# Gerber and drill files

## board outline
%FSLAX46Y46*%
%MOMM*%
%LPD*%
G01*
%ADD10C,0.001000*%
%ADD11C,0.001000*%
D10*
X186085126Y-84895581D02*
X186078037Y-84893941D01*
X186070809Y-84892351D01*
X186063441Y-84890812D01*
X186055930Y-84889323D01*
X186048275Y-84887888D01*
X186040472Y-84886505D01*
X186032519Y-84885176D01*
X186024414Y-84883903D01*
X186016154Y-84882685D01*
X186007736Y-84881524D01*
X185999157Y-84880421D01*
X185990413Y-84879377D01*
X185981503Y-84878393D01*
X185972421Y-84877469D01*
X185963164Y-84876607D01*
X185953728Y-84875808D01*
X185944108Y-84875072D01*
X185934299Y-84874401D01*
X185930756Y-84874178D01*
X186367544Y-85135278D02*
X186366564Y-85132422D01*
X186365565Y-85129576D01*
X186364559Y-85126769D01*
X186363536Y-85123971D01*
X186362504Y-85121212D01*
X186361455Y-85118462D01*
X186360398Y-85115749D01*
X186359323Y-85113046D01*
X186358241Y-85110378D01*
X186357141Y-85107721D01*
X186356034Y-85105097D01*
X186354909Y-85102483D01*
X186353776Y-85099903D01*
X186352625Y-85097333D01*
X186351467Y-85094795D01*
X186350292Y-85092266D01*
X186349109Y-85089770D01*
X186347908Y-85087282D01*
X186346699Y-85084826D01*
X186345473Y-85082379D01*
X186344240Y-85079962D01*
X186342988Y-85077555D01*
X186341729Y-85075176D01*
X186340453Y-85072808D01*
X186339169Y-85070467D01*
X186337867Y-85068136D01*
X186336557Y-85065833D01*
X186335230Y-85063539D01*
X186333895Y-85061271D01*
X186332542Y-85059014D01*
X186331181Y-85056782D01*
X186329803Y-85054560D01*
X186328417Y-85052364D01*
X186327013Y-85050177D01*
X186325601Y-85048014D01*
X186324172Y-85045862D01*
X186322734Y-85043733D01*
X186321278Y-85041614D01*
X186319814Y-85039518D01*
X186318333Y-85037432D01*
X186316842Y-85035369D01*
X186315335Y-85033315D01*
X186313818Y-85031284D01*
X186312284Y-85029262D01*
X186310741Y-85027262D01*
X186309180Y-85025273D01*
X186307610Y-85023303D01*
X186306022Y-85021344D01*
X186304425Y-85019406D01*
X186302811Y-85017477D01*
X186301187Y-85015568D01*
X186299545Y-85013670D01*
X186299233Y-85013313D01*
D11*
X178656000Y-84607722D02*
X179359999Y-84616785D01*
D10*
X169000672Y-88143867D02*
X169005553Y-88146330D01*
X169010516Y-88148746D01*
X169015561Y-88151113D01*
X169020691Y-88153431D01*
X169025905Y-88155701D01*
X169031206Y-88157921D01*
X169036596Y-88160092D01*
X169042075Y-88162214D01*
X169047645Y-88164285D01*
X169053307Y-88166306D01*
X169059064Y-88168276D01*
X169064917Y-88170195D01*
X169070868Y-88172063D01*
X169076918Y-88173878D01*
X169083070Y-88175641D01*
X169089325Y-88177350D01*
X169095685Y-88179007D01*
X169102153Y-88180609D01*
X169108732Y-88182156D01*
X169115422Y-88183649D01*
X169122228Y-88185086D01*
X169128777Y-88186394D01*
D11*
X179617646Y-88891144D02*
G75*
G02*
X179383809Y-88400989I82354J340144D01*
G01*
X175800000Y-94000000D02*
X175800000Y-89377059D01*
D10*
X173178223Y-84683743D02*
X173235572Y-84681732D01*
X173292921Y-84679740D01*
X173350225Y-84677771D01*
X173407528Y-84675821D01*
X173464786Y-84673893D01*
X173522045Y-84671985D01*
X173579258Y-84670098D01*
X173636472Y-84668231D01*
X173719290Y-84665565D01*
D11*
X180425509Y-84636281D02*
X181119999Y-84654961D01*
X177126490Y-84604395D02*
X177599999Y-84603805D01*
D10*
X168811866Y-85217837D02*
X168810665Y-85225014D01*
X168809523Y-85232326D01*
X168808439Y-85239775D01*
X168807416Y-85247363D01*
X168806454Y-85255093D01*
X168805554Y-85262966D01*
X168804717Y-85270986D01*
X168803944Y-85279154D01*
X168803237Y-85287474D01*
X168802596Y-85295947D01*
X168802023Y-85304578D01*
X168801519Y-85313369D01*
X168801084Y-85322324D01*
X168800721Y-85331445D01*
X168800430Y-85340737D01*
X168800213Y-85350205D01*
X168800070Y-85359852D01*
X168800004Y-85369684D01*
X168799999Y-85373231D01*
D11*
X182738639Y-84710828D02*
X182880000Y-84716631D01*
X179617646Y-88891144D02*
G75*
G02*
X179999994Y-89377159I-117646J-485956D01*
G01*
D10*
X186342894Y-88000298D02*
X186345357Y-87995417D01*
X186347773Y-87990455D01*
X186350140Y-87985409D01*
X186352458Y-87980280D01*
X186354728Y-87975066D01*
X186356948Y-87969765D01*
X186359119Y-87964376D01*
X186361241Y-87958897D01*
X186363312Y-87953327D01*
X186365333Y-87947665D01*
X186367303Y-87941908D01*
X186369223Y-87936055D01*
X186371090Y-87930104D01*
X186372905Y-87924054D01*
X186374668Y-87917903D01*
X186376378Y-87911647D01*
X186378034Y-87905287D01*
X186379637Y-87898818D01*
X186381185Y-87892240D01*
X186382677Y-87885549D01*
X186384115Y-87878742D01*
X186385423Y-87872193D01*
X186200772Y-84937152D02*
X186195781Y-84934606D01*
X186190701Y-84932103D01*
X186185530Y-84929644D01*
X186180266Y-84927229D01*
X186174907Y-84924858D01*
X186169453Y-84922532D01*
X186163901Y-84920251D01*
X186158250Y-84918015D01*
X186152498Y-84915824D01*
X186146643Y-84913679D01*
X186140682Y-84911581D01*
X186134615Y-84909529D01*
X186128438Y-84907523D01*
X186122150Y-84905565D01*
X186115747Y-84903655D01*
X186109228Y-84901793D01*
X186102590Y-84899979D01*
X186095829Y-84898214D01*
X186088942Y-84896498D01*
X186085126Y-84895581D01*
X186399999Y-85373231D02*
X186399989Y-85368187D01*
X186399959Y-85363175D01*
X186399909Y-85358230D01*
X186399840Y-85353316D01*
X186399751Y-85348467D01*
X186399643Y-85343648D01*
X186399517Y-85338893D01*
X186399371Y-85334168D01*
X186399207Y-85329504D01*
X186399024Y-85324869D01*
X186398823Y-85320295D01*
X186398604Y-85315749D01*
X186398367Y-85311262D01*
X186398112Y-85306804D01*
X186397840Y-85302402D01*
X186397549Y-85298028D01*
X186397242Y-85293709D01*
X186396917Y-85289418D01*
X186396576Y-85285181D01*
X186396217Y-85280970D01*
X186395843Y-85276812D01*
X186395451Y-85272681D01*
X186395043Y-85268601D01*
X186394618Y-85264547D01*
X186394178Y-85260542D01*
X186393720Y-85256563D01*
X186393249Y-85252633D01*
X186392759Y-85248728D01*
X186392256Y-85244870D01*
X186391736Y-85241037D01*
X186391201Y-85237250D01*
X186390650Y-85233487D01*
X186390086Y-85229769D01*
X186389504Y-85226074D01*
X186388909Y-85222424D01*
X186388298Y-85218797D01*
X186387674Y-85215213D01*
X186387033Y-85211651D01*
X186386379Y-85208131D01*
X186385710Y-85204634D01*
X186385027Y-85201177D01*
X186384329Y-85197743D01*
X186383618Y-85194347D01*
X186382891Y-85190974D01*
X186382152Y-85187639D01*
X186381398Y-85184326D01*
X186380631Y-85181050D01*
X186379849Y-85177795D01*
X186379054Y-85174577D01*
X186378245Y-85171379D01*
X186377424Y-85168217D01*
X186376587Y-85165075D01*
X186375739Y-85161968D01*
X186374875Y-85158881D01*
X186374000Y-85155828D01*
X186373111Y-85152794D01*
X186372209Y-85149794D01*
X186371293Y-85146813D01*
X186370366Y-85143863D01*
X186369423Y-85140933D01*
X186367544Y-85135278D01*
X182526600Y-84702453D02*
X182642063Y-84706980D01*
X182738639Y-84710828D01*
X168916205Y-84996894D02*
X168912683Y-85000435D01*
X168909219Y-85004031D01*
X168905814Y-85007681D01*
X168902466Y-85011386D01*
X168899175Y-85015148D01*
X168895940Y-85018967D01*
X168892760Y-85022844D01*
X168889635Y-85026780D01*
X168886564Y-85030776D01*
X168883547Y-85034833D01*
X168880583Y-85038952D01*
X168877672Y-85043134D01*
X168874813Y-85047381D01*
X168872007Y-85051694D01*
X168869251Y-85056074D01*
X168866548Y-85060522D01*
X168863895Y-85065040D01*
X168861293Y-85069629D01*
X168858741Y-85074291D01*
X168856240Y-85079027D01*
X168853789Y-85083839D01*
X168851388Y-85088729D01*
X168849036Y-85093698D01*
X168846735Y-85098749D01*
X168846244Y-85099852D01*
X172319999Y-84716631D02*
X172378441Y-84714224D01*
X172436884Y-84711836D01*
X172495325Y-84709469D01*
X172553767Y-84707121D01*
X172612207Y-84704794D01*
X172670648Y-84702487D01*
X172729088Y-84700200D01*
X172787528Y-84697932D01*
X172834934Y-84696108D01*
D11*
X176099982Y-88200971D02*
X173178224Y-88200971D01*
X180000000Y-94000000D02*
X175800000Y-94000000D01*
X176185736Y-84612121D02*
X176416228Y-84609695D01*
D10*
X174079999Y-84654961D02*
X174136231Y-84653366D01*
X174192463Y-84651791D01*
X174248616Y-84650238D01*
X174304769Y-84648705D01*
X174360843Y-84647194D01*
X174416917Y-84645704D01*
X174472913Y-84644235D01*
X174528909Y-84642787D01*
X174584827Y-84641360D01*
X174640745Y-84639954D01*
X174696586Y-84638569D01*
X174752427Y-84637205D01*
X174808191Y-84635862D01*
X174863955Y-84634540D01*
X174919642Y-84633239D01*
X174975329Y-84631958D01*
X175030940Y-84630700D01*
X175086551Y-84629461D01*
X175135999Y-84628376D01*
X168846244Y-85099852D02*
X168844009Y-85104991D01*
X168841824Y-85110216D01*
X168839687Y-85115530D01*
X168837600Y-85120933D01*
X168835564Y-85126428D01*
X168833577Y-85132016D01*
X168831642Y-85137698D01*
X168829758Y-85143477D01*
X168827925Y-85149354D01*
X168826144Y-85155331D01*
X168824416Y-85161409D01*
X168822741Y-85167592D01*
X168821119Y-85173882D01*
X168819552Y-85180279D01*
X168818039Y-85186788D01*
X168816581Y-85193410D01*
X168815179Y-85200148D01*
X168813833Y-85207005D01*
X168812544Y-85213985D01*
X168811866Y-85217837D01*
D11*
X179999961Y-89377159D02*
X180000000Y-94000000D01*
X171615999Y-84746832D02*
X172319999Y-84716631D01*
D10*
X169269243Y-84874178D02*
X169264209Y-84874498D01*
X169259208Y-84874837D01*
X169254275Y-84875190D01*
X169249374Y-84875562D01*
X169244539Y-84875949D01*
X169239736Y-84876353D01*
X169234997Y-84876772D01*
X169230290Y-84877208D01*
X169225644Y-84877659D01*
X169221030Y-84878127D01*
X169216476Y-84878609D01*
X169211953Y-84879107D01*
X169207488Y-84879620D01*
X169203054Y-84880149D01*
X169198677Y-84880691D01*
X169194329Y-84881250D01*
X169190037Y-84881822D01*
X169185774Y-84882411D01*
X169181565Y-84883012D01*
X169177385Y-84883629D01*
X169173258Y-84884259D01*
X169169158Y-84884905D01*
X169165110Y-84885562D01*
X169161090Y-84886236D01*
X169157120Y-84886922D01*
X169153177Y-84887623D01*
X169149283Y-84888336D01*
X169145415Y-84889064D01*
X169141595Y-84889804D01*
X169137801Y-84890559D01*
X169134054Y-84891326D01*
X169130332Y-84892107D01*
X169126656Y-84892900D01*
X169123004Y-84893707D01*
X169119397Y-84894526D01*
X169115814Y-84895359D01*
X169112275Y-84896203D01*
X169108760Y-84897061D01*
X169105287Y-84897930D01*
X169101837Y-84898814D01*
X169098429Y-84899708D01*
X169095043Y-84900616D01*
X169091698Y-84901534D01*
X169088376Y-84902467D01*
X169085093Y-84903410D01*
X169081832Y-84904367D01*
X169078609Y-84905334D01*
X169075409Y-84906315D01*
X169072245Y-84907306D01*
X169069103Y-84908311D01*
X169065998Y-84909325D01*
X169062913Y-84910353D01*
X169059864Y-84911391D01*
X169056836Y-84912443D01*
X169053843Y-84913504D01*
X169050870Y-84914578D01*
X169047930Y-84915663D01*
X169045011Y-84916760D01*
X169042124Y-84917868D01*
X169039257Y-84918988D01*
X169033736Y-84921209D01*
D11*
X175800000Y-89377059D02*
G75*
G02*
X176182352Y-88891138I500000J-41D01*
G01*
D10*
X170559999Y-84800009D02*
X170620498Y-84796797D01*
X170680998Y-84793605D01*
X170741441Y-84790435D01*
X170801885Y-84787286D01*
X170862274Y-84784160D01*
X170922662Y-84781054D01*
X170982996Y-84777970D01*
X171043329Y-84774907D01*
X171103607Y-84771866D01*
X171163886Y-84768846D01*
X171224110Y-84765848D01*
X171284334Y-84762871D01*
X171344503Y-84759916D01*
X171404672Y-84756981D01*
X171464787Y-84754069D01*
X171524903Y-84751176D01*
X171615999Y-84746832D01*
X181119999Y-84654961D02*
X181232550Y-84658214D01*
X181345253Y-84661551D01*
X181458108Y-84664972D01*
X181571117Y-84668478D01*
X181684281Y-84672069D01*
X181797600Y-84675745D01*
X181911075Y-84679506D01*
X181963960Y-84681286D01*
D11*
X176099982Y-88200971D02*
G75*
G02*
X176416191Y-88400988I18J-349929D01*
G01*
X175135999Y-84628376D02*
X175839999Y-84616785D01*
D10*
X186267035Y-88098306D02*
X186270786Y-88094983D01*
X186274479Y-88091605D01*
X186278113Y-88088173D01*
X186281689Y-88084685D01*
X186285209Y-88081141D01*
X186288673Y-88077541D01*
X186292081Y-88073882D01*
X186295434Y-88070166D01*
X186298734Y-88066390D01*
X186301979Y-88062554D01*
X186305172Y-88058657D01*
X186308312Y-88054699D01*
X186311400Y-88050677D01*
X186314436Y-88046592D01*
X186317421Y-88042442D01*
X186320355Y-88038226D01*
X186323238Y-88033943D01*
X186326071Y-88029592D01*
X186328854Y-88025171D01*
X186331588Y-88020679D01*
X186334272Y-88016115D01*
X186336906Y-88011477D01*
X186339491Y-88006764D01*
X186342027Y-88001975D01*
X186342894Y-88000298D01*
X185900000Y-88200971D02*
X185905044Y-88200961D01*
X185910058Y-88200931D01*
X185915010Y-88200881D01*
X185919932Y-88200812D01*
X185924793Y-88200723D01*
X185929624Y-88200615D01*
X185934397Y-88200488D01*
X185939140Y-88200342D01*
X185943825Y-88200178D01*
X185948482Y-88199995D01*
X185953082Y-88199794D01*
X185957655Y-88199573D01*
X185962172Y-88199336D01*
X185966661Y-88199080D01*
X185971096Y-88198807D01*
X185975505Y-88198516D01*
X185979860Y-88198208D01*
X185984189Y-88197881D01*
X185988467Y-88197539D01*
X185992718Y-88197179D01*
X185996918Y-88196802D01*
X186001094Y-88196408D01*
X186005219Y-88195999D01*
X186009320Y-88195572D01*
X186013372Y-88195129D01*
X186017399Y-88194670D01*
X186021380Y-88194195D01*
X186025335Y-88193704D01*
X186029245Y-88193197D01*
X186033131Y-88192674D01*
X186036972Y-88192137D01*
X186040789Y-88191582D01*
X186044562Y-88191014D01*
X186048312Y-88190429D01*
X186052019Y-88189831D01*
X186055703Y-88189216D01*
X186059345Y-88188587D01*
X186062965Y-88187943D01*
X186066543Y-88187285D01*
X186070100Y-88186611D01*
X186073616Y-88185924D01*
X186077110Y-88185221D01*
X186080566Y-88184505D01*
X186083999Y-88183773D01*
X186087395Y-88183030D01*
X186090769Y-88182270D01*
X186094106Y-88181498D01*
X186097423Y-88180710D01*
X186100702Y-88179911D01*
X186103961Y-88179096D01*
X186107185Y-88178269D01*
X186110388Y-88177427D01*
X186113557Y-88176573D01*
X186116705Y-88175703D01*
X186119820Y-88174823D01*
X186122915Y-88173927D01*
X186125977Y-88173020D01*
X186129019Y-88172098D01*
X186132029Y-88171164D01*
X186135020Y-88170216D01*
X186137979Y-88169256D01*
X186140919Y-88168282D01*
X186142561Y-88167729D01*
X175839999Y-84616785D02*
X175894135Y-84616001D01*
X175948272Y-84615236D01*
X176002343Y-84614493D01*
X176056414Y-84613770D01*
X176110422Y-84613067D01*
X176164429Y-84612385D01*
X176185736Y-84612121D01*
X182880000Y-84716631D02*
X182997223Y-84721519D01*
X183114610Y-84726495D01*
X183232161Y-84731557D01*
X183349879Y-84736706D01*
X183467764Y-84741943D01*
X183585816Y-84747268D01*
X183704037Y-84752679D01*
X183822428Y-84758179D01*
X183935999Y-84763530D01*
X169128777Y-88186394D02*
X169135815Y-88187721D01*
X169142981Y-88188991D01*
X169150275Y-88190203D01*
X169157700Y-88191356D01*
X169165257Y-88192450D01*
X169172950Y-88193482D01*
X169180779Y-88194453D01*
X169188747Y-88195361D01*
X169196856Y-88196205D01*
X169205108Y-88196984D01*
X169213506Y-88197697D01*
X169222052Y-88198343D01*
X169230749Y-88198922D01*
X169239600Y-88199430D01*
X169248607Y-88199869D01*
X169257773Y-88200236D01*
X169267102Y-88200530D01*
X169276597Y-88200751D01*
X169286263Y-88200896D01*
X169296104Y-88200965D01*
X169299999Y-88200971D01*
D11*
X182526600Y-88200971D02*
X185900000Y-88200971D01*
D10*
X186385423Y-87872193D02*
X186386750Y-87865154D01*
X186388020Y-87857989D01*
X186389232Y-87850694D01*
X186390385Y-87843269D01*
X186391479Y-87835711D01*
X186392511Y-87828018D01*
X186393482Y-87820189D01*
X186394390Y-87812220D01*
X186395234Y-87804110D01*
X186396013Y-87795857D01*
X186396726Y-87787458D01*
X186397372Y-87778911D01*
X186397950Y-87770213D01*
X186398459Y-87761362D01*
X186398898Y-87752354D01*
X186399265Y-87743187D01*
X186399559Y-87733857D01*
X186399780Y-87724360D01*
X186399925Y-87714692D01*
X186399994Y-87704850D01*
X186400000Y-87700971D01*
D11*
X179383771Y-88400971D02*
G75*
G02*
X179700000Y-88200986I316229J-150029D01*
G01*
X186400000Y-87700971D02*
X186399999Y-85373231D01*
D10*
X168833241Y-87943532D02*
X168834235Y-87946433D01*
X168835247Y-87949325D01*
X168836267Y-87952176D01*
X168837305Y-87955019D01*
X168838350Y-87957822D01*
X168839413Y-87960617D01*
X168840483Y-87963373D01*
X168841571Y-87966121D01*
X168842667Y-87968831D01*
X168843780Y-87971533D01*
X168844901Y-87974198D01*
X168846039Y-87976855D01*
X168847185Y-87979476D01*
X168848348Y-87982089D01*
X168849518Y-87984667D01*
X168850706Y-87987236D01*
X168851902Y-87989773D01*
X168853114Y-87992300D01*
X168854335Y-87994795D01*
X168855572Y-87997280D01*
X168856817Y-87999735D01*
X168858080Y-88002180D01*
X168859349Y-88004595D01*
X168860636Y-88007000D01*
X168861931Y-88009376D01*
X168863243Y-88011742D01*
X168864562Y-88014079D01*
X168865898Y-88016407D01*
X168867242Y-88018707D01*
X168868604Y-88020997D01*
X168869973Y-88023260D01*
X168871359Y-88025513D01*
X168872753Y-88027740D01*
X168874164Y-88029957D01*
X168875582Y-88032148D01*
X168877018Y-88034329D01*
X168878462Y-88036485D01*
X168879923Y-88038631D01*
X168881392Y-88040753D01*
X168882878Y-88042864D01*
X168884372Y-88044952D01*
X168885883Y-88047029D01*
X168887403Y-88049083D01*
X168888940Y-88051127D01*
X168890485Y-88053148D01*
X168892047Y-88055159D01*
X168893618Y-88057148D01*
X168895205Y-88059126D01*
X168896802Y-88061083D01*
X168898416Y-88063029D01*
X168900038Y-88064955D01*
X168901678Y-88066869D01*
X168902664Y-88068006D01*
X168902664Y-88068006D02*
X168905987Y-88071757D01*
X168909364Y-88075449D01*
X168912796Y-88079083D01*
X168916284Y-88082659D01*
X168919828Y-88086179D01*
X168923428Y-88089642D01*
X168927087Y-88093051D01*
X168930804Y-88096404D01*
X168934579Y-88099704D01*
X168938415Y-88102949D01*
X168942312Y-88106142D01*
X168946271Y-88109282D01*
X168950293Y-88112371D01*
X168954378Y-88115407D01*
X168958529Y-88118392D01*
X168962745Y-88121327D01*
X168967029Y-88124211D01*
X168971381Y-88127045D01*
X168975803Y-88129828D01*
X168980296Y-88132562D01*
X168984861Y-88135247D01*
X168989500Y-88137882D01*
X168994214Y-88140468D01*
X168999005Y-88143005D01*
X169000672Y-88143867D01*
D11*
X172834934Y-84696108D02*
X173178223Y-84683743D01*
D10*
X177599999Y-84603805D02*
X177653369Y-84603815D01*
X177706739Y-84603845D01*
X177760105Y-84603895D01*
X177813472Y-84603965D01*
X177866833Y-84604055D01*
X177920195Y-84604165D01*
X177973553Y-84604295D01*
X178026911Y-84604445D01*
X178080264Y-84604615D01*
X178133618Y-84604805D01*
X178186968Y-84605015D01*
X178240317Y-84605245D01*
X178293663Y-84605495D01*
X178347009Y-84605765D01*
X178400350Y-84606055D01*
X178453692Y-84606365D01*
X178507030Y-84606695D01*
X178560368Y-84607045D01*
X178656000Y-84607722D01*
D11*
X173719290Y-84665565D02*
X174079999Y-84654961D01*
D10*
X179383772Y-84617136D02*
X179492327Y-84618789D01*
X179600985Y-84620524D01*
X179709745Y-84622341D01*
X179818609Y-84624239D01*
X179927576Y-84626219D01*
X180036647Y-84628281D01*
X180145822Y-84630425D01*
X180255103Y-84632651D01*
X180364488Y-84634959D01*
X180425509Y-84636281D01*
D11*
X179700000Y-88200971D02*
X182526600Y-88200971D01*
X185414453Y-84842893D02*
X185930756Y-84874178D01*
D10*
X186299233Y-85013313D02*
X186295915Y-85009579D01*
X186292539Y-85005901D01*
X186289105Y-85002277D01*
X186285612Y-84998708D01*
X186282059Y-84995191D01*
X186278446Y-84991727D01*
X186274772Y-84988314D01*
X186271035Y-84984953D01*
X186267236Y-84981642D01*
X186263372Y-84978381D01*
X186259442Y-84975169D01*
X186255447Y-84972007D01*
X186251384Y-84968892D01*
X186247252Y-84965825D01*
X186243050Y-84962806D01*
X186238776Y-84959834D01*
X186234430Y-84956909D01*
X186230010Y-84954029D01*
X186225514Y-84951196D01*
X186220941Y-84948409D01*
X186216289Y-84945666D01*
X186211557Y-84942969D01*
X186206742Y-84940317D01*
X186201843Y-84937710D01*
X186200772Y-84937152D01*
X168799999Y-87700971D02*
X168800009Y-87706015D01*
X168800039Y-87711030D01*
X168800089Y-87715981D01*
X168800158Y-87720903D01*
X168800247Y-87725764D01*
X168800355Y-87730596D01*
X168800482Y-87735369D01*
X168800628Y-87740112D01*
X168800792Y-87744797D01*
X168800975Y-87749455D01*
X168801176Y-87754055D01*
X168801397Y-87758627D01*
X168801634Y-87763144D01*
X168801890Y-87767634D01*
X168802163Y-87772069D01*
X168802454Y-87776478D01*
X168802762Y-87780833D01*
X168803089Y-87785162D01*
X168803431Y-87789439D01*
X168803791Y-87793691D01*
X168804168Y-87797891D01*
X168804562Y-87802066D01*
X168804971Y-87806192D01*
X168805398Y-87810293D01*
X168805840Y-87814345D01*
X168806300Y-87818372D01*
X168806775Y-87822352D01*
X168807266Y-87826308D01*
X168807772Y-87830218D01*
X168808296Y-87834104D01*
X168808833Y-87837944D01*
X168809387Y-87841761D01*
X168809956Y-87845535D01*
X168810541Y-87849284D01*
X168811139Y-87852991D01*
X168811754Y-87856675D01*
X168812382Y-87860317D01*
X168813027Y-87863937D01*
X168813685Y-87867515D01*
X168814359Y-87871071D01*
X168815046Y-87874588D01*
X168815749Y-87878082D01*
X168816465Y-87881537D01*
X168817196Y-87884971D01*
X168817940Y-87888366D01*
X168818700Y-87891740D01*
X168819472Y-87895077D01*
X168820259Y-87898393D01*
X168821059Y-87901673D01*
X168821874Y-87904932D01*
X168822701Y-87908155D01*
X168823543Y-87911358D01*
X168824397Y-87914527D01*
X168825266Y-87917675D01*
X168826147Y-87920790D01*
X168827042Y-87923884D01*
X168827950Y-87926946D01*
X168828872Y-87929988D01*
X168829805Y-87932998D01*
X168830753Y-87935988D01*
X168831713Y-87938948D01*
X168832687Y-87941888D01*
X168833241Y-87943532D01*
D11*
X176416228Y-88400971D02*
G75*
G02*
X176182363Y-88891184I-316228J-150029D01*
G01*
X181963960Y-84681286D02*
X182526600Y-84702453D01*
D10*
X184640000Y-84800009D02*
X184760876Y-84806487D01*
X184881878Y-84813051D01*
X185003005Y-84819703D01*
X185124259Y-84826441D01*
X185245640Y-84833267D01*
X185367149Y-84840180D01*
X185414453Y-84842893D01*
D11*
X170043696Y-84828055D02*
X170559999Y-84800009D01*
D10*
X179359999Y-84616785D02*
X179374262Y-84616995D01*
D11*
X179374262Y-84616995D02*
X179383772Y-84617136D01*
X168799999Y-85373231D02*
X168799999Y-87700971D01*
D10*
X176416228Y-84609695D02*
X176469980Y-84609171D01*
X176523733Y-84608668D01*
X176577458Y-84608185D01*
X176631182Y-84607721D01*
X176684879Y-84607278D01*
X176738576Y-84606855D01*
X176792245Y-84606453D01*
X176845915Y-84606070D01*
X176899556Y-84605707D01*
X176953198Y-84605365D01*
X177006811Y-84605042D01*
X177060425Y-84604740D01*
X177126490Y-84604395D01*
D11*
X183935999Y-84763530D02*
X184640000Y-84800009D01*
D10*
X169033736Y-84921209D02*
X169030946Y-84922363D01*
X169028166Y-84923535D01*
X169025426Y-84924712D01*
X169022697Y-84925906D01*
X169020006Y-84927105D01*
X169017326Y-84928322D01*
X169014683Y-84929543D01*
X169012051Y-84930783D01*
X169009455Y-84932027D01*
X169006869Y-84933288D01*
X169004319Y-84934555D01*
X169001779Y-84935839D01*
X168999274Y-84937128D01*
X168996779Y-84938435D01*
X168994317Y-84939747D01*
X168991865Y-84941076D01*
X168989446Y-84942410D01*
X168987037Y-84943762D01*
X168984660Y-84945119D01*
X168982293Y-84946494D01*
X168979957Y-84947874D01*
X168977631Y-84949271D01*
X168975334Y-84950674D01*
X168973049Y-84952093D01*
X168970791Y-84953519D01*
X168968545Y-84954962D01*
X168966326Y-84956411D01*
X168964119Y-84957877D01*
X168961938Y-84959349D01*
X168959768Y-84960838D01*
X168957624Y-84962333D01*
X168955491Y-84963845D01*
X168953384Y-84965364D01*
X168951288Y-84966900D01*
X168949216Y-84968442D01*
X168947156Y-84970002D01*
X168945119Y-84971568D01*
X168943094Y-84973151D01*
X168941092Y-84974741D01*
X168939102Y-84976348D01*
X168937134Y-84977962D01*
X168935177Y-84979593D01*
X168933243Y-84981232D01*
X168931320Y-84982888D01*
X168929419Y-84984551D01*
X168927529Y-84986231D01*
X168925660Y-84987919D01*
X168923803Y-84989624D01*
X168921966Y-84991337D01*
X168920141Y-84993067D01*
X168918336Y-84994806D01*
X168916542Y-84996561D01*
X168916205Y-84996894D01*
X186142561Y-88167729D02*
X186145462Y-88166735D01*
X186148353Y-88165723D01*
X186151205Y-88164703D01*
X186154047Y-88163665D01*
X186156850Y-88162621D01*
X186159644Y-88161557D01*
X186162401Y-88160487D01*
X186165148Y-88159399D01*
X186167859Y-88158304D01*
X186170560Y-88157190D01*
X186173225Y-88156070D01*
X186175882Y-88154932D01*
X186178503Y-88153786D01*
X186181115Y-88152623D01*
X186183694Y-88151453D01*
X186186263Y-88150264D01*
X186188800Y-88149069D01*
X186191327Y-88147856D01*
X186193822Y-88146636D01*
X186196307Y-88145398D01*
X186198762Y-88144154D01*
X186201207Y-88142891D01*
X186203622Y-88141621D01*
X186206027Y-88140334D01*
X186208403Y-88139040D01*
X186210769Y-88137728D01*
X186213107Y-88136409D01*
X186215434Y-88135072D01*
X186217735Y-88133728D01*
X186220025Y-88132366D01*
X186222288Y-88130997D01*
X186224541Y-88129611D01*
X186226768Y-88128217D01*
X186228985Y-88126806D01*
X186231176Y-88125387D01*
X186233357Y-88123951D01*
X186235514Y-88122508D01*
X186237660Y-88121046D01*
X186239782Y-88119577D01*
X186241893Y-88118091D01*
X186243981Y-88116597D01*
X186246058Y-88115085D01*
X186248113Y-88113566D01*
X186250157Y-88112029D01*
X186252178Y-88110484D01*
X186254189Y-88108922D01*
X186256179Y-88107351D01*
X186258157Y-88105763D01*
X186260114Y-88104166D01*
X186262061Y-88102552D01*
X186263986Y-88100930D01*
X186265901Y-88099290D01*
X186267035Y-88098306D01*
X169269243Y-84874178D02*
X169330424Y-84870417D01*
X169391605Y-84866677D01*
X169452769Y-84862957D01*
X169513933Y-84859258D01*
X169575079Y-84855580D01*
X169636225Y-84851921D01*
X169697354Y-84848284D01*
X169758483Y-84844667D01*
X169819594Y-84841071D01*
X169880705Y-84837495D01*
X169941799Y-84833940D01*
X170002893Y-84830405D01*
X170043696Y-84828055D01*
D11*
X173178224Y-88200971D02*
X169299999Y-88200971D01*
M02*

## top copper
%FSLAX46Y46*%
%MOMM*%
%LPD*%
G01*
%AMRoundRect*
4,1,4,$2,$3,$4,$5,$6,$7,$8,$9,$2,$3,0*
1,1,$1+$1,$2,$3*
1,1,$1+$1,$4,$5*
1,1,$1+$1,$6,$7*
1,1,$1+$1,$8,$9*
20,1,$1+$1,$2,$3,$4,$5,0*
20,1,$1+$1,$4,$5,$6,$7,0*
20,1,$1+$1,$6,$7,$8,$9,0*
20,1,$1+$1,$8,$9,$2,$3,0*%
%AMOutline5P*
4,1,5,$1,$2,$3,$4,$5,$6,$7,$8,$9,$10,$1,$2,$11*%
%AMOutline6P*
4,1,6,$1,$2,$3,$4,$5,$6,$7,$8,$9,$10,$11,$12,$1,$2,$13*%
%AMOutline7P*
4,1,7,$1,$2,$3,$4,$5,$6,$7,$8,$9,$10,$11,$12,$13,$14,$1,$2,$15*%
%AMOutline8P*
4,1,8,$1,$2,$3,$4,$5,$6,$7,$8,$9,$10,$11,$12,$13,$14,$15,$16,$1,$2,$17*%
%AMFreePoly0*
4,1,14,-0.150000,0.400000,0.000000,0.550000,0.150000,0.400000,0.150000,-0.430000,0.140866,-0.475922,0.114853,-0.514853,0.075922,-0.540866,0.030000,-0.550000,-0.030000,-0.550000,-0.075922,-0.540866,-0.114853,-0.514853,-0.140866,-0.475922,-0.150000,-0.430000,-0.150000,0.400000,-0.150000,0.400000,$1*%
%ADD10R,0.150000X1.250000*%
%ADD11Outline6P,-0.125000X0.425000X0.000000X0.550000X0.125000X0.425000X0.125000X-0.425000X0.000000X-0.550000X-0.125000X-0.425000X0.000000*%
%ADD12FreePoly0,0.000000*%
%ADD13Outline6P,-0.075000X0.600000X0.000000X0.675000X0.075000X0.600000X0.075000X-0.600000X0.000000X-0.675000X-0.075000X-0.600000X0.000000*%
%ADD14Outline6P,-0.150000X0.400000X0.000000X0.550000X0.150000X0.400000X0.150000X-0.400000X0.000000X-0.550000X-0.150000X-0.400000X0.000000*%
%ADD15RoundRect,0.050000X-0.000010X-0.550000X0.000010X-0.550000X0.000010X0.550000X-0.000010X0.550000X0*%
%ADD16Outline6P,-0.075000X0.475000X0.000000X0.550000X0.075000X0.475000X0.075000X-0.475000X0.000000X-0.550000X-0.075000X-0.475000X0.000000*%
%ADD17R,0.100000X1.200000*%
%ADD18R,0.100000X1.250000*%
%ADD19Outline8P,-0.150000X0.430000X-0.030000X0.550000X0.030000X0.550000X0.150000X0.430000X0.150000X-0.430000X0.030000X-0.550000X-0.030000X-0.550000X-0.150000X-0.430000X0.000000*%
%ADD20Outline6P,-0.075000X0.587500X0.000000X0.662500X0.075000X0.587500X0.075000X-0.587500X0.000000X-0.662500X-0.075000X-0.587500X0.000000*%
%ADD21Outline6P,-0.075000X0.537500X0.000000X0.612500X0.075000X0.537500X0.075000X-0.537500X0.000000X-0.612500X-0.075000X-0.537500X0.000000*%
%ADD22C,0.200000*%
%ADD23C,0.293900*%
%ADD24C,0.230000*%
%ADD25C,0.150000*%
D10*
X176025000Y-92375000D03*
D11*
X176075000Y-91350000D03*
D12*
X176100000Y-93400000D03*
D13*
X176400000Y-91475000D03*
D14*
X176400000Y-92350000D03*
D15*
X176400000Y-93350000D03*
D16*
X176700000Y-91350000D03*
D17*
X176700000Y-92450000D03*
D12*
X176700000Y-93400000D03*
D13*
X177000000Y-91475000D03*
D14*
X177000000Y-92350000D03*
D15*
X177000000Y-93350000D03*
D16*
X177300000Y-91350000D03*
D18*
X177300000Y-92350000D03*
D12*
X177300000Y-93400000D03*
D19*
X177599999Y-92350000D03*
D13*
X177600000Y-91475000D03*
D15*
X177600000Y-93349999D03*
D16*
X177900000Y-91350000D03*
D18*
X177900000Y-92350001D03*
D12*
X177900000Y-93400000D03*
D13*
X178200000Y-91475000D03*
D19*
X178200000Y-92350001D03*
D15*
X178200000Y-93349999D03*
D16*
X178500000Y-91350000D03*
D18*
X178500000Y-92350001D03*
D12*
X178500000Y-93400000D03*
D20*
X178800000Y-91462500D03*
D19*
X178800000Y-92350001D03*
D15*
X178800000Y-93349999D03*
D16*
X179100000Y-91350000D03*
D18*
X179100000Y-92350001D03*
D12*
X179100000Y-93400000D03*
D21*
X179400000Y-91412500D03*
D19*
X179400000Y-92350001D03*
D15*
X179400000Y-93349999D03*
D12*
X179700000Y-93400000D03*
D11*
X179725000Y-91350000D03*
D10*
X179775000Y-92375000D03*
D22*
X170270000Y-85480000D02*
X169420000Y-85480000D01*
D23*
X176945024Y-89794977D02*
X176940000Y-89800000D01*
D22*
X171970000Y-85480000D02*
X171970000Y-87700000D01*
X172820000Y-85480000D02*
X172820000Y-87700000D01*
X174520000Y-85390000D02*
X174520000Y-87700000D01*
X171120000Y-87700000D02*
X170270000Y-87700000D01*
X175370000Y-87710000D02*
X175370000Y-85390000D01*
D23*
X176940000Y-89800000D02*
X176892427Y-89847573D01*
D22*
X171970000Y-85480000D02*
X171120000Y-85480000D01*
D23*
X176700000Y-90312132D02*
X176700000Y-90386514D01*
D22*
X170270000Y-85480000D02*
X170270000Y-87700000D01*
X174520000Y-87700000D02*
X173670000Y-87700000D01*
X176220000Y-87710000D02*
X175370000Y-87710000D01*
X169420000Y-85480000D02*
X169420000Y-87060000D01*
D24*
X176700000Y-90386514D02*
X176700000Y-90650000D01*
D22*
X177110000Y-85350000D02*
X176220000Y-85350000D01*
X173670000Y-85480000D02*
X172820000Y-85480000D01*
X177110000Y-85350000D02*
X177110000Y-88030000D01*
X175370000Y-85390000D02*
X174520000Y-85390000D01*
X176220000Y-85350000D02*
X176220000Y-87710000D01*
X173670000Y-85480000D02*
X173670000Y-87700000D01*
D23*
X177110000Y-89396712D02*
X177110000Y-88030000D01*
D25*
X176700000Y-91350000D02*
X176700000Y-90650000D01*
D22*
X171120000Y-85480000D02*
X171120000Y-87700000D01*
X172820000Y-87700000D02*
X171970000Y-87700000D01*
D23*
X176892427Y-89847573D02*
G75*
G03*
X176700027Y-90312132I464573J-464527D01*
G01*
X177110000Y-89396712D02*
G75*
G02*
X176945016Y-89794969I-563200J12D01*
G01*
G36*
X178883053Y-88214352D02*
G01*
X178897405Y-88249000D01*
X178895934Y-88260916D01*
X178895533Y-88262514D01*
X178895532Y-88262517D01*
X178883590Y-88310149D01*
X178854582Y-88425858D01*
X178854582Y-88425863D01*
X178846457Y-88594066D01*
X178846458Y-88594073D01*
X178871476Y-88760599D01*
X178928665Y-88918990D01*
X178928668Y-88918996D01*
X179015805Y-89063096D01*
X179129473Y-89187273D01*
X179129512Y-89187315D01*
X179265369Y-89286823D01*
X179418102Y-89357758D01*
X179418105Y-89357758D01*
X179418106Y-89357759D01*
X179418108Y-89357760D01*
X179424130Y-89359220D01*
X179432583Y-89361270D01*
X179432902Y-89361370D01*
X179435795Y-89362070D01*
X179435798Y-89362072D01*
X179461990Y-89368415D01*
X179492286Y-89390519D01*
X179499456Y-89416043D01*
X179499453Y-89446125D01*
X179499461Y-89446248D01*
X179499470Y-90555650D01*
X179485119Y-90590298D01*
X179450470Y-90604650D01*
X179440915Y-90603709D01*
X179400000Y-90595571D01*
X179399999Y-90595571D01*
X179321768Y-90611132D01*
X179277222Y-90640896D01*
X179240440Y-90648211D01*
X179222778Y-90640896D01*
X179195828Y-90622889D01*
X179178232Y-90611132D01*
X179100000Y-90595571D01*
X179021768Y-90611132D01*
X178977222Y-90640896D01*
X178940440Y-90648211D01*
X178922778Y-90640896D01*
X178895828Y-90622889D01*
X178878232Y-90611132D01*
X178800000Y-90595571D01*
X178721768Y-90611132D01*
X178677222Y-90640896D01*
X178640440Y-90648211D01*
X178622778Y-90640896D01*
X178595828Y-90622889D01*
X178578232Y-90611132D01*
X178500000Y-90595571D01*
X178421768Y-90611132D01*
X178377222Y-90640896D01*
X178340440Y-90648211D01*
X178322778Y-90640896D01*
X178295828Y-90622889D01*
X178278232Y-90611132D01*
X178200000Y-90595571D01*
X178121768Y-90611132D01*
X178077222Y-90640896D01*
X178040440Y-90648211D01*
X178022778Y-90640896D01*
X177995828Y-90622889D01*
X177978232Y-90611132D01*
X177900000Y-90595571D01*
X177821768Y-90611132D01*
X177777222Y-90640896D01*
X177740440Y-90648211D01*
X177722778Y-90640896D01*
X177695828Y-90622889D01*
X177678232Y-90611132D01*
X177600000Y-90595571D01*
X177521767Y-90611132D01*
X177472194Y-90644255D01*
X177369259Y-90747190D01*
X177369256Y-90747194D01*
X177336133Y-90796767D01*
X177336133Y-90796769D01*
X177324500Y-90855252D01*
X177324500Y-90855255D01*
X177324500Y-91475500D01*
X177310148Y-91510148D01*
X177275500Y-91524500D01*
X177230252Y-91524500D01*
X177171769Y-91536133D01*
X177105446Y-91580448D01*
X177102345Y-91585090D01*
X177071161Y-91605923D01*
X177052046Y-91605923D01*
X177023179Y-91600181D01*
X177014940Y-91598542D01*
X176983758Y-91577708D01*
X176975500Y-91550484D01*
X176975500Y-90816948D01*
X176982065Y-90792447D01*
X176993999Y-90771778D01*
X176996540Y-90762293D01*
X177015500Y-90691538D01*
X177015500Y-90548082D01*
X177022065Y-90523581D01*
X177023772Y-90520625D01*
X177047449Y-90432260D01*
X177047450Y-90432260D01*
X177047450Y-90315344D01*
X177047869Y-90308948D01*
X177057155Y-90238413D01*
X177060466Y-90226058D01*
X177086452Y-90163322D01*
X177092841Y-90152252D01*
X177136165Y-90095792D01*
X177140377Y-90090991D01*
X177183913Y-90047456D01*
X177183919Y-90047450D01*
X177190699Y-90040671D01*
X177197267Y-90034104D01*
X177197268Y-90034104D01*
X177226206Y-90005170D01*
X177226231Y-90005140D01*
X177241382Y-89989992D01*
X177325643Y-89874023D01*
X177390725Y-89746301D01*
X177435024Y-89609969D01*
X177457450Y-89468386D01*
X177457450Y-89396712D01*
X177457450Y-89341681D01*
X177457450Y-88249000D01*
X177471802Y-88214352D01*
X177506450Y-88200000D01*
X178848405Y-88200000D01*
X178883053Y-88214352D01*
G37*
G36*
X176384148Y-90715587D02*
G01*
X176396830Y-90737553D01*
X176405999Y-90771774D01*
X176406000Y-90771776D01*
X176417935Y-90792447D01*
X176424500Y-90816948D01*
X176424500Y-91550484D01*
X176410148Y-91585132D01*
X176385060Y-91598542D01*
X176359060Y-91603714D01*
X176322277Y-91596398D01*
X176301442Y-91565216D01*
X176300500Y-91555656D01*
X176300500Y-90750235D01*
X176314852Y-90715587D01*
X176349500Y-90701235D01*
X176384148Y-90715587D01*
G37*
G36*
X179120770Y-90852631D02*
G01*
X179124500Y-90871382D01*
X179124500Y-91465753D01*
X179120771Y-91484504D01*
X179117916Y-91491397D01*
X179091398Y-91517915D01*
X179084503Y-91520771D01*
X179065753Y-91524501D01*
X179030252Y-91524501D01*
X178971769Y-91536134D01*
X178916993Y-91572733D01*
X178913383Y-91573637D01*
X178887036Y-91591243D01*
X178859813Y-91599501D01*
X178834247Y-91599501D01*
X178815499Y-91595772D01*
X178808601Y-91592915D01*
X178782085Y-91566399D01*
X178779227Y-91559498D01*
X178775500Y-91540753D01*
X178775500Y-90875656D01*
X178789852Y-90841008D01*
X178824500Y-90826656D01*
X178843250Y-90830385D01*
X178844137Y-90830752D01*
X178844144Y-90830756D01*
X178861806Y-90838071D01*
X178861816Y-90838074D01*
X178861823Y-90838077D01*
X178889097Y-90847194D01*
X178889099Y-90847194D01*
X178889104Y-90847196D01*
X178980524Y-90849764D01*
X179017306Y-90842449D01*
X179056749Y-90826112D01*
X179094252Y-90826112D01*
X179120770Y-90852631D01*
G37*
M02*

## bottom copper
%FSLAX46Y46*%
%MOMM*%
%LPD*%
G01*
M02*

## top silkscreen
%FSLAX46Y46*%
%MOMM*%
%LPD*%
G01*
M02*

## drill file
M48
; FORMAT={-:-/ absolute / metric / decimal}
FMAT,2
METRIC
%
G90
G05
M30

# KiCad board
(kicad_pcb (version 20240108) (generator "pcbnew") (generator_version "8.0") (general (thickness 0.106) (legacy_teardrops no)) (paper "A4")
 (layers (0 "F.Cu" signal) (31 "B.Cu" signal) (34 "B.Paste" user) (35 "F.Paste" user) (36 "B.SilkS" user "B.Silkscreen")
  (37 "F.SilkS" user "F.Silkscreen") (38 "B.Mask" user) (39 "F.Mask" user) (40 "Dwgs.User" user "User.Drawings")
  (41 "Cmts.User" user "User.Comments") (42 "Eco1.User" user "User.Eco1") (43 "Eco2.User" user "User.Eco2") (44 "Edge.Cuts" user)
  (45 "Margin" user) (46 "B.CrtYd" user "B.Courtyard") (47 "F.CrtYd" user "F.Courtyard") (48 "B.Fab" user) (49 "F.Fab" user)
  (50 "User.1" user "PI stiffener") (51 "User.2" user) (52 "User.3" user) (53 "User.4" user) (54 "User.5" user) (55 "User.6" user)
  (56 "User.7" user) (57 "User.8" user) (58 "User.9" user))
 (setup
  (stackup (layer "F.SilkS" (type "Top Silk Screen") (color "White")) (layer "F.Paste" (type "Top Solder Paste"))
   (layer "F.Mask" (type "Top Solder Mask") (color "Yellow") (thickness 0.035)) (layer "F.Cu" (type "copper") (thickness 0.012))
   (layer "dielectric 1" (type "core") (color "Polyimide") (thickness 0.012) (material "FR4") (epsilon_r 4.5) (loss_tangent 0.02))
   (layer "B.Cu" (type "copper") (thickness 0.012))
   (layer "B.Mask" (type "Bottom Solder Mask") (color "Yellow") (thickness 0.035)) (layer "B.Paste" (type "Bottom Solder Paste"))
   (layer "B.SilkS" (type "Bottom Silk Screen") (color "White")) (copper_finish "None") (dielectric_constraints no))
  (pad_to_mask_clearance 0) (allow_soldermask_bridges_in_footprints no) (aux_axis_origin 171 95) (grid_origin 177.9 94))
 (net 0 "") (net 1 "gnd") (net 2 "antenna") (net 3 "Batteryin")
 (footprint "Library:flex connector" (layer "B.Cu") (at 175.7 90.05)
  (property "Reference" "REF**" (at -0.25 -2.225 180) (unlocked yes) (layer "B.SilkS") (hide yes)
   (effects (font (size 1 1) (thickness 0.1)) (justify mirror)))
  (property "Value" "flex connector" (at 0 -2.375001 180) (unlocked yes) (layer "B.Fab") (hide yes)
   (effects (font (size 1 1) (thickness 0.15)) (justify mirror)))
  (pad "1" smd rect (at 0.325 2.325) (size 0.15 1.25) (layers "F.Cu" "F.Paste" "F.Mask") (thermal_bridge_angle 45))
  (pad "1" smd roundrect (at 0.375 1.3) (size 0.25 1.1) (layers "F.Cu" "F.Paste" "F.Mask") (roundrect_rratio 0) (chamfer_ratio 0.5)
   (chamfer top_left top_right bottom_left bottom_right) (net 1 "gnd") (thermal_bridge_angle 45))
  (pad "1" smd roundrect (at 0.4 3.35) (size 0.3 1.1) (layers "F.Cu" "F.Paste" "F.Mask") (roundrect_rratio 0.4) (chamfer_ratio 0.5)
   (chamfer top_left top_right) (thermal_bridge_angle 45))
  (pad "2" smd roundrect (at 0.7 1.425) (size 0.15 1.35) (layers "F.Cu" "F.Paste" "F.Mask") (roundrect_rratio 0) (chamfer_ratio 0.5)
   (chamfer top_left top_right bottom_left bottom_right) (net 1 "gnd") (thermal_bridge_angle 45))
  (pad "2" smd roundrect (at 0.7 2.3) (size 0.3 1.1) (layers "F.Cu" "F.Paste" "F.Mask") (roundrect_rratio 0) (chamfer_ratio 0.5)
   (chamfer top_left top_right bottom_left bottom_right) (thermal_bridge_angle 45))
  (pad "2" smd roundrect (at 0.7 3.3) (size 0.1 1.2) (layers "F.Cu" "F.Paste" "F.Mask") (roundrect_rratio 0.5) (thermal_bridge_angle 45))
  (pad "3" smd roundrect (at 1 1.3) (size 0.15 1.1) (layers "F.Cu" "F.Paste" "F.Mask") (roundrect_rratio 0) (chamfer_ratio 0.5)
   (chamfer top_left top_right bottom_left bottom_right) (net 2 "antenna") (thermal_bridge_angle 45))
  (pad "3" smd rect (at 1 2.4) (size 0.1 1.2) (layers "F.Cu" "F.Paste" "F.Mask") (thermal_bridge_angle 45))
  (pad "3" smd roundrect (at 1 3.35) (size 0.3 1.1) (layers "F.Cu" "F.Paste" "F.Mask") (roundrect_rratio 0.4) (chamfer_ratio 0.5)
   (chamfer top_left top_right) (thermal_bridge_angle 45))
  (pad "4" smd roundrect (at 1.3 1.425) (size 0.15 1.35) (layers "F.Cu" "F.Paste" "F.Mask") (roundrect_rratio 0) (chamfer_ratio 0.5)
   (chamfer top_left top_right bottom_left bottom_right) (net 1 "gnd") (thermal_bridge_angle 45))
  (pad "4" smd roundrect (at 1.3 2.3) (size 0.3 1.1) (layers "F.Cu" "F.Paste" "F.Mask") (roundrect_rratio 0) (chamfer_ratio 0.5)
   (chamfer top_left top_right bottom_left bottom_right) (thermal_bridge_angle 45))
  (pad "4" smd roundrect (at 1.3 3.3) (size 0.1 1.2) (layers "F.Cu" "F.Paste" "F.Mask") (roundrect_rratio 0.5) (thermal_bridge_angle 45))
  (pad "5" smd roundrect (at 1.6 1.3) (size 0.15 1.1) (layers "F.Cu" "F.Paste" "F.Mask") (roundrect_rratio 0) (chamfer_ratio 0.5)
   (chamfer top_left top_right bottom_left bottom_right) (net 1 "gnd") (thermal_bridge_angle 45))
  (pad "5" smd rect (at 1.6 2.3) (size 0.1 1.25) (layers "F.Cu" "F.Paste" "F.Mask") (thermal_bridge_angle 45))
  (pad "5" smd roundrect (at 1.6 3.35) (size 0.3 1.1) (layers "F.Cu" "F.Paste" "F.Mask") (roundrect_rratio 0.4) (chamfer_ratio 0.5)
   (chamfer top_left top_right) (thermal_bridge_angle 45))
  (pad "6" smd roundrect (at 1.899999 2.3) (size 0.3 1.1) (layers "F.Cu" "F.Paste" "F.Mask") (roundrect_rratio 0) (chamfer_ratio 0.4)
   (chamfer top_left top_right bottom_left bottom_right) (thermal_bridge_angle 45))
  (pad "6" smd roundrect (at 1.9 1.425) (size 0.15 1.35) (layers "F.Cu" "F.Paste" "F.Mask") (roundrect_rratio 0) (chamfer_ratio 0.5)
   (chamfer top_left top_right bottom_left bottom_right) (thermal_bridge_angle 45))
  (pad "6" smd roundrect (at 1.9 3.299999) (size 0.1 1.2) (layers "F.Cu" "F.Paste" "F.Mask") (roundrect_rratio 0.5)
   (thermal_bridge_angle 45))
  (pad "7" smd roundrect (at 2.2 1.3) (size 0.15 1.1) (layers "F.Cu" "F.Paste" "F.Mask") (roundrect_rratio 0) (chamfer_ratio 0.5)
   (chamfer top_left top_right bottom_left bottom_right) (thermal_bridge_angle 45))
  (pad "7" smd rect (at 2.2 2.300001) (size 0.1 1.25) (layers "F.Cu" "F.Paste" "F.Mask") (thermal_bridge_angle 45))
  (pad "7" smd roundrect (at 2.2 3.35) (size 0.3 1.1) (layers "F.Cu" "F.Paste" "F.Mask") (roundrect_rratio 0.4) (chamfer_ratio 0.5)
   (chamfer top_left top_right) (thermal_bridge_angle 45))
  (pad "8" smd roundrect (at 2.5 1.425) (size 0.15 1.35) (layers "F.Cu" "F.Paste" "F.Mask") (roundrect_rratio 0) (chamfer_ratio 0.5)
   (chamfer top_left top_right bottom_left bottom_right) (thermal_bridge_angle 45))
  (pad "8" smd roundrect (at 2.5 2.300001) (size 0.3 1.1) (layers "F.Cu" "F.Paste" "F.Mask") (roundrect_rratio 0) (chamfer_ratio 0.4)
   (chamfer top_left top_right bottom_left bottom_right) (thermal_bridge_angle 45))
  (pad "8" smd roundrect (at 2.5 3.299999) (size 0.1 1.2) (layers "F.Cu" "F.Paste" "F.Mask") (roundrect_rratio 0.5)
   (thermal_bridge_angle 45))
  (pad "9" smd roundrect (at 2.8 1.3) (size 0.15 1.1) (layers "F.Cu" "F.Paste" "F.Mask") (roundrect_rratio 0) (chamfer_ratio 0.5)
   (chamfer top_left top_right bottom_left bottom_right) (thermal_bridge_angle 45))
  (pad "9" smd rect (at 2.8 2.300001) (size 0.1 1.25) (layers "F.Cu" "F.Paste" "F.Mask") (thermal_bridge_angle 45))
  (pad "9" smd roundrect (at 2.8 3.35) (size 0.3 1.1) (layers "F.Cu" "F.Paste" "F.Mask") (roundrect_rratio 0.4) (chamfer_ratio 0.5)
   (chamfer top_left top_right) (thermal_bridge_angle 45))
  (pad "10" smd roundrect (at 3.1 1.4125) (size 0.15 1.325) (layers "F.Cu" "F.Paste" "F.Mask") (roundrect_rratio 0) (chamfer_ratio 0.5)
   (chamfer top_left top_right bottom_left bottom_right) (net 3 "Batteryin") (thermal_bridge_angle 45))
  (pad "10" smd roundrect (at 3.1 2.300001) (size 0.3 1.1) (layers "F.Cu" "F.Paste" "F.Mask") (roundrect_rratio 0) (chamfer_ratio 0.4)
   (chamfer top_left top_right bottom_left bottom_right) (thermal_bridge_angle 45))
  (pad "10" smd roundrect (at 3.1 3.299999) (size 0.1 1.2) (layers "F.Cu" "F.Paste" "F.Mask") (roundrect_rratio 0.5)
   (thermal_bridge_angle 45))
  (pad "11" smd roundrect (at 3.4 1.3) (size 0.15 1.1) (layers "F.Cu" "F.Paste" "F.Mask") (roundrect_rratio 0) (chamfer_ratio 0.5)
   (chamfer top_left top_right bottom_left bottom_right) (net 3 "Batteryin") (thermal_bridge_angle 45))
  (pad "11" smd rect (at 3.4 2.300001) (size 0.1 1.25) (layers "F.Cu" "F.Paste" "F.Mask") (thermal_bridge_angle 45))
  (pad "11" smd roundrect (at 3.4 3.35) (size 0.3 1.1) (layers "F.Cu" "F.Paste" "F.Mask") (roundrect_rratio 0.4) (chamfer_ratio 0.5)
   (chamfer top_left top_right) (thermal_bridge_angle 45))
  (pad "12" smd roundrect (at 3.7 1.3625) (size 0.15 1.225) (layers "F.Cu" "F.Paste" "F.Mask") (roundrect_rratio 0) (chamfer_ratio 0.5)
   (chamfer top_left top_right bottom_left bottom_right) (thermal_bridge_angle 45))
  (pad "12" smd roundrect (at 3.7 2.300001) (size 0.3 1.1) (layers "F.Cu" "F.Paste" "F.Mask") (roundrect_rratio 0) (chamfer_ratio 0.4)
   (chamfer top_left top_right bottom_left bottom_right) (thermal_bridge_angle 45))
  (pad "12" smd roundrect (at 3.7 3.299999) (size 0.1 1.2) (layers "F.Cu" "F.Paste" "F.Mask") (roundrect_rratio 0.5)
   (thermal_bridge_angle 45))
  (pad "13" smd roundrect (at 4 3.35) (size 0.3 1.1) (layers "F.Cu" "F.Paste" "F.Mask") (roundrect_rratio 0.4) (chamfer_ratio 0.5)
   (chamfer top_left top_right) (thermal_bridge_angle 45))
  (pad "13" smd roundrect (at 4.025 1.3) (size 0.25 1.1) (layers "F.Cu" "F.Paste" "F.Mask") (roundrect_rratio 0) (chamfer_ratio 0.5)
   (chamfer top_left top_right bottom_left bottom_right) (thermal_bridge_angle 45))
  (pad "13" smd rect (at 4.075 2.325) (size 0.15 1.25) (layers "F.Cu" "F.Paste" "F.Mask") (thermal_bridge_angle 45)))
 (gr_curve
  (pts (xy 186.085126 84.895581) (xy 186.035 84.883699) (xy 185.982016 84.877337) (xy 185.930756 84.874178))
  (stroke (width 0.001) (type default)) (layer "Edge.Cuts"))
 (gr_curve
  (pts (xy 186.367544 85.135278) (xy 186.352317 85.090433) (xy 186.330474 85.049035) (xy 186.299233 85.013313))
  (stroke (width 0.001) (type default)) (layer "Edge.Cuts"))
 (gr_line (start 178.656 84.607722) (end 179.359999 84.616785) (stroke (width 0.001) (type default)) (layer "Edge.Cuts"))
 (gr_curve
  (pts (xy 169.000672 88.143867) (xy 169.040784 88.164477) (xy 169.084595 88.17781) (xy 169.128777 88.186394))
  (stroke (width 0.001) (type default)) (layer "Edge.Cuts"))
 (gr_arc (start 179.617646 88.891144) (mid 179.384095 88.70169) (end 179.383771 88.400971) (stroke (width 0.001) (type default))
  (layer "Edge.Cuts"))
 (gr_line (start 175.8 94) (end 175.8 89.377059) (stroke (width 0.001) (type default)) (layer "Edge.Cuts"))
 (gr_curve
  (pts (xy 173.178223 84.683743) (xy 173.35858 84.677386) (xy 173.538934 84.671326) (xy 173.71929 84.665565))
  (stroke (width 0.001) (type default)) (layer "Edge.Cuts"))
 (gr_line (start 180.425509 84.636281) (end 181.119999 84.654961) (stroke (width 0.001) (type default)) (layer "Edge.Cuts"))
 (gr_line (start 177.12649 84.604395) (end 177.599999 84.603805) (stroke (width 0.001) (type default)) (layer "Edge.Cuts"))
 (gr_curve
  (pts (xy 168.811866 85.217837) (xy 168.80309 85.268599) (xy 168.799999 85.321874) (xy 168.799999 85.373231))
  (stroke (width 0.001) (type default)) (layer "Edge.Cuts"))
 (gr_line (start 182.738639 84.710828) (end 182.88 84.716631) (stroke (width 0.001) (type default)) (layer "Edge.Cuts"))
 (gr_arc (start 179.617646 88.891144) (mid 179.892941 89.067961) (end 179.999961 89.377159) (stroke (width 0.001) (type default))
  (layer "Edge.Cuts"))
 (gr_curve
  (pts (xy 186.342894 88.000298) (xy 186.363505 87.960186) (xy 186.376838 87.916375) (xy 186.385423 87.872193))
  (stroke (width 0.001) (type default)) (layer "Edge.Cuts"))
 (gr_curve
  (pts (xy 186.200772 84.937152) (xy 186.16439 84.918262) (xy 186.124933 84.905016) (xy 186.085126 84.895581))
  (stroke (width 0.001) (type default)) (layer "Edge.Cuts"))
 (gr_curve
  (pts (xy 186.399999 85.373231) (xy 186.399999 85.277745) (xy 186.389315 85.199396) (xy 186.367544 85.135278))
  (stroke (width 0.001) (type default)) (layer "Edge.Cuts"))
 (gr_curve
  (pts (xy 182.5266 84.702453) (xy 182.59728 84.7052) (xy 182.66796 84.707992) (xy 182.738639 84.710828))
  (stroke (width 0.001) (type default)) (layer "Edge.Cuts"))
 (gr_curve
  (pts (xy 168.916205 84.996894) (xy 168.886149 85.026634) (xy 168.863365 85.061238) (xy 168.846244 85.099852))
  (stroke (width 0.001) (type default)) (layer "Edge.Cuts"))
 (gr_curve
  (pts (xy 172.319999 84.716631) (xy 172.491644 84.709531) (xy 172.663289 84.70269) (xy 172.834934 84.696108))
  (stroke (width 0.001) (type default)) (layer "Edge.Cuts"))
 (gr_line (start 176.099982 88.200971) (end 173.178224 88.200971) (stroke (width 0.001) (type default)) (layer "Edge.Cuts"))
 (gr_line (start 180 94) (end 175.8 94) (stroke (width 0.001) (type default)) (layer "Edge.Cuts"))
 (gr_line (start 176.185736 84.612121) (end 176.416228 84.609695) (stroke (width 0.001) (type default)) (layer "Edge.Cuts"))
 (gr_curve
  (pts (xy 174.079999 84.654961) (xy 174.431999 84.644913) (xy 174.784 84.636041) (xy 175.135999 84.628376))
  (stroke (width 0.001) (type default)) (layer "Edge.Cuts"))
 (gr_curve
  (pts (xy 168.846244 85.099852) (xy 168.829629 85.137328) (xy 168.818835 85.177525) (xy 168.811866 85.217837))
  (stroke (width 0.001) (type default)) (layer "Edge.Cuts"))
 (gr_line (start 179.999961 89.377159) (end 180 94) (stroke (width 0.001) (type default)) (layer "Edge.Cuts"))
 (gr_line (start 171.615999 84.746832) (end 172.319999 84.716631) (stroke (width 0.001) (type default)) (layer "Edge.Cuts"))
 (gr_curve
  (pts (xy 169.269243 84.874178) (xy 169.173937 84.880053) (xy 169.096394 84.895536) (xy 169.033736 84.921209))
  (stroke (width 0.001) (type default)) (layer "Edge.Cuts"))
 (gr_arc (start 175.8 89.377059) (mid 175.907054 89.067918) (end 176.182353 88.891144) (stroke (width 0.001) (type default))
  (layer "Edge.Cuts"))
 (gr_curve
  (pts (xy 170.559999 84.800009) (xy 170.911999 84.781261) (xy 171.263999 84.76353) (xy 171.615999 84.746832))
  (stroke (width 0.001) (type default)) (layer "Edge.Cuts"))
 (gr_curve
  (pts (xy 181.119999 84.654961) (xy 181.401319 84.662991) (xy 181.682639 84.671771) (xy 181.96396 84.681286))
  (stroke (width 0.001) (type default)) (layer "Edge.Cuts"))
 (gr_arc (start 176.099982 88.200971) (mid 176.287082 88.255161) (end 176.416228 88.400971) (stroke (width 0.001) (type default))
  (layer "Edge.Cuts"))
 (gr_line (start 175.135999 84.628376) (end 175.839999 84.616785) (stroke (width 0.001) (type default)) (layer "Edge.Cuts"))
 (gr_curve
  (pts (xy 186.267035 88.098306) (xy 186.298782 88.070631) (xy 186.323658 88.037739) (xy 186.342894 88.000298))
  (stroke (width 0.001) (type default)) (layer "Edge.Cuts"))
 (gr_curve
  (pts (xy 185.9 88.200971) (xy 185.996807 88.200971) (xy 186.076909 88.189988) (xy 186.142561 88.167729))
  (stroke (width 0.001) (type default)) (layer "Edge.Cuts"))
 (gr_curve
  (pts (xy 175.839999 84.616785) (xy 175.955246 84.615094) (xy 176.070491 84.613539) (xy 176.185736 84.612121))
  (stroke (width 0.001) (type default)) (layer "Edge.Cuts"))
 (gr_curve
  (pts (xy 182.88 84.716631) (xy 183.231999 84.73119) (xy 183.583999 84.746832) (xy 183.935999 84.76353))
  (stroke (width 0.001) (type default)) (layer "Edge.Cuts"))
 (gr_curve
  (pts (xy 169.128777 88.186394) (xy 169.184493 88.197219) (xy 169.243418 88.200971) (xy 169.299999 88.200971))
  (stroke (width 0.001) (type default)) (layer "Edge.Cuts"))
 (gr_line (start 182.5266 88.200971) (end 185.9 88.200971) (stroke (width 0.001) (type default)) (layer "Edge.Cuts"))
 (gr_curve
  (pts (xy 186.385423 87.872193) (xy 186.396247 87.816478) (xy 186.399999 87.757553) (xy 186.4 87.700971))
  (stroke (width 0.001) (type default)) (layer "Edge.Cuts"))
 (gr_arc (start 179.383771 88.400971) (mid 179.512916 88.255168) (end 179.7 88.200971) (stroke (width 0.001) (type default))
  (layer "Edge.Cuts"))
 (gr_line (start 186.4 87.700971) (end 186.399999 85.373231) (stroke (width 0.001) (type default)) (layer "Edge.Cuts"))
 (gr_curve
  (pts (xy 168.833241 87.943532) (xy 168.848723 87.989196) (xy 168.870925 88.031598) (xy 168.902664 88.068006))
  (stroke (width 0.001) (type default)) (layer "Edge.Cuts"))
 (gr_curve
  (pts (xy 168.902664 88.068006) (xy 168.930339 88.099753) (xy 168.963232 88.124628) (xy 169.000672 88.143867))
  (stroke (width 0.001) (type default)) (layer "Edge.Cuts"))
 (gr_line (start 172.834934 84.696108) (end 173.178223 84.683743) (stroke (width 0.001) (type default)) (layer "Edge.Cuts"))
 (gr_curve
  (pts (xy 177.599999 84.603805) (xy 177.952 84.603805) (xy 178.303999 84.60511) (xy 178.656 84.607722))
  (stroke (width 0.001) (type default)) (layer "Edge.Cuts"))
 (gr_line (start 173.71929 84.665565) (end 174.079999 84.654961) (stroke (width 0.001) (type default)) (layer "Edge.Cuts"))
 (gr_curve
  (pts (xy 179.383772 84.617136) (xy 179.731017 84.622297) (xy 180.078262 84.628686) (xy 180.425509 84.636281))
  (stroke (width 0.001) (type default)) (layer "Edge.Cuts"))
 (gr_line (start 179.7 88.200971) (end 182.5266 88.200971) (stroke (width 0.001) (type default)) (layer "Edge.Cuts"))
 (gr_line (start 185.414453 84.842893) (end 185.930756 84.874178) (stroke (width 0.001) (type default)) (layer "Edge.Cuts"))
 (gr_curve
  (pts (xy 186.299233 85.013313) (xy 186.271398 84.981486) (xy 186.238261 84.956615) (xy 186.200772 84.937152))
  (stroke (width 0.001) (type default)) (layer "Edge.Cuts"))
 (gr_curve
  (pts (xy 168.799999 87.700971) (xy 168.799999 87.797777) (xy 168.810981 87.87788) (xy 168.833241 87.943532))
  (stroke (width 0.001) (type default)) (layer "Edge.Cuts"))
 (gr_arc (start 176.416228 88.400971) (mid 176.415878 88.701683) (end 176.182353 88.891144) (stroke (width 0.001) (type default))
  (layer "Edge.Cuts"))
 (gr_line (start 181.96396 84.681286) (end 182.5266 84.702453) (stroke (width 0.001) (type default)) (layer "Edge.Cuts"))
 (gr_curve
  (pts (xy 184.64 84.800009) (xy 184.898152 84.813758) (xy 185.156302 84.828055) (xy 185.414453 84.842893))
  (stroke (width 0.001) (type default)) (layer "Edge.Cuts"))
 (gr_line (start 170.043696 84.828055) (end 170.559999 84.800009) (stroke (width 0.001) (type default)) (layer "Edge.Cuts"))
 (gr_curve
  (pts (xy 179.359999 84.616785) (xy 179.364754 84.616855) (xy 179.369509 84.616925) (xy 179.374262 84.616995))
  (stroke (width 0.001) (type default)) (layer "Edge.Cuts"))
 (gr_line (start 179.374262 84.616995) (end 179.383772 84.617136) (stroke (width 0.001) (type default)) (layer "Edge.Cuts"))
 (gr_line (start 168.799999 85.373231) (end 168.799999 87.700971) (stroke (width 0.001) (type default)) (layer "Edge.Cuts"))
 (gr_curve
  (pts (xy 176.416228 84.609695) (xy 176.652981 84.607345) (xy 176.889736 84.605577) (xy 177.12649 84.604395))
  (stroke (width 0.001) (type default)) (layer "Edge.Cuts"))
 (gr_line (start 183.935999 84.76353) (end 184.64 84.800009) (stroke (width 0.001) (type default)) (layer "Edge.Cuts"))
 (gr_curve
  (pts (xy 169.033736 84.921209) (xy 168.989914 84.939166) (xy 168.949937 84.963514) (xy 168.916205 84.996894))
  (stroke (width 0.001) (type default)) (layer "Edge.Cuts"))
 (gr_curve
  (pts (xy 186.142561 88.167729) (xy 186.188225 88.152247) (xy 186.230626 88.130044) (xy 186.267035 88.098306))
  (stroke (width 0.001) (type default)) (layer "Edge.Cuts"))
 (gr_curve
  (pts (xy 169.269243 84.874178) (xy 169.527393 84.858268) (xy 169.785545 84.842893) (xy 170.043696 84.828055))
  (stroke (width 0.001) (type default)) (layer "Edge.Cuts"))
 (gr_line (start 173.178224 88.200971) (end 169.299999 88.200971) (stroke (width 0.001) (type default)) (layer "Edge.Cuts"))
 (segment (start 170.27 85.48) (end 169.42 85.48) (width 0.2) (layer "F.Cu") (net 2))
 (segment (start 176.945024 89.794977) (end 176.94 89.8) (width 0.2939) (layer "F.Cu") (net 2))
 (segment (start 171.97 85.48) (end 171.97 87.7) (width 0.2) (layer "F.Cu") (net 2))
 (segment (start 172.82 85.48) (end 172.82 87.7) (width 0.2) (layer "F.Cu") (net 2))
 (segment (start 174.52 85.39) (end 174.52 87.7) (width 0.2) (layer "F.Cu") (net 2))
 (segment (start 171.12 87.7) (end 170.27 87.7) (width 0.2) (layer "F.Cu") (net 2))
 (segment (start 175.37 87.71) (end 175.37 85.39) (width 0.2) (layer "F.Cu") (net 2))
 (segment (start 176.94 89.8) (end 176.892427 89.847573) (width 0.2939) (layer "F.Cu") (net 2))
 (segment (start 171.97 85.48) (end 171.12 85.48) (width 0.2) (layer "F.Cu") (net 2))
 (segment (start 176.7 90.312132) (end 176.7 90.386514) (width 0.2939) (layer "F.Cu") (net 2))
 (segment (start 170.27 85.48) (end 170.27 87.7) (width 0.2) (layer "F.Cu") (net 2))
 (segment (start 174.52 87.7) (end 173.67 87.7) (width 0.2) (layer "F.Cu") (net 2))
 (segment (start 176.22 87.71) (end 175.37 87.71) (width 0.2) (layer "F.Cu") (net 2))
 (segment (start 169.42 85.48) (end 169.42 87.06) (width 0.2) (layer "F.Cu") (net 2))
 (segment (start 176.7 90.386514) (end 176.7 90.65) (width 0.23) (layer "F.Cu") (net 2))
 (segment (start 177.11 85.35) (end 176.22 85.35) (width 0.2) (layer "F.Cu") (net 2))
 (segment (start 173.67 85.48) (end 172.82 85.48) (width 0.2) (layer "F.Cu") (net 2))
 (segment (start 177.11 85.35) (end 177.11 88.03) (width 0.2) (layer "F.Cu") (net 2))
 (segment (start 175.37 85.39) (end 174.52 85.39) (width 0.2) (layer "F.Cu") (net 2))
 (segment (start 176.22 85.35) (end 176.22 87.71) (width 0.2) (layer "F.Cu") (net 2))
 (segment (start 173.67 85.48) (end 173.67 87.7) (width 0.2) (layer "F.Cu") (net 2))
 (segment (start 177.11 89.396712) (end 177.11 88.03) (width 0.2939) (layer "F.Cu") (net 2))
 (segment (start 176.7 91.35) (end 176.7 90.65) (width 0.15) (layer "F.Cu") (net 2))
 (segment (start 171.12 85.48) (end 171.12 87.7) (width 0.2) (layer "F.Cu") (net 2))
 (segment (start 172.82 87.7) (end 171.97 87.7) (width 0.2) (layer "F.Cu") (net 2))
 (arc (start 176.892427 89.847573) (mid 176.75001 90.060714) (end 176.7 90.312132) (width 0.2939) (layer "F.Cu") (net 2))
 (arc (start 177.11 89.396712) (mid 177.067134 89.612229) (end 176.945024 89.794977) (width 0.2939) (layer "F.Cu") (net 2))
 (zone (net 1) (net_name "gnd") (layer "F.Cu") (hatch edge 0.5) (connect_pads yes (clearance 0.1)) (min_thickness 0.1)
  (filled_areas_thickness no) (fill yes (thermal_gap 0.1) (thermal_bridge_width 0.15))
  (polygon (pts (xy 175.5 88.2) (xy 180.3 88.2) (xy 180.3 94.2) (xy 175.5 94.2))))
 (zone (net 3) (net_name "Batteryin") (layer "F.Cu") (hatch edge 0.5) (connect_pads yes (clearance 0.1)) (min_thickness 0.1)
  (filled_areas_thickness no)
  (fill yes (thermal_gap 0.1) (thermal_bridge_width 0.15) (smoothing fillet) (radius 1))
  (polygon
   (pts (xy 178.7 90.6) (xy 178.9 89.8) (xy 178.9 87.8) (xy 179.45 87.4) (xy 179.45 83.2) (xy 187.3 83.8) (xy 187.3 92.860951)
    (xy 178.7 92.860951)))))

